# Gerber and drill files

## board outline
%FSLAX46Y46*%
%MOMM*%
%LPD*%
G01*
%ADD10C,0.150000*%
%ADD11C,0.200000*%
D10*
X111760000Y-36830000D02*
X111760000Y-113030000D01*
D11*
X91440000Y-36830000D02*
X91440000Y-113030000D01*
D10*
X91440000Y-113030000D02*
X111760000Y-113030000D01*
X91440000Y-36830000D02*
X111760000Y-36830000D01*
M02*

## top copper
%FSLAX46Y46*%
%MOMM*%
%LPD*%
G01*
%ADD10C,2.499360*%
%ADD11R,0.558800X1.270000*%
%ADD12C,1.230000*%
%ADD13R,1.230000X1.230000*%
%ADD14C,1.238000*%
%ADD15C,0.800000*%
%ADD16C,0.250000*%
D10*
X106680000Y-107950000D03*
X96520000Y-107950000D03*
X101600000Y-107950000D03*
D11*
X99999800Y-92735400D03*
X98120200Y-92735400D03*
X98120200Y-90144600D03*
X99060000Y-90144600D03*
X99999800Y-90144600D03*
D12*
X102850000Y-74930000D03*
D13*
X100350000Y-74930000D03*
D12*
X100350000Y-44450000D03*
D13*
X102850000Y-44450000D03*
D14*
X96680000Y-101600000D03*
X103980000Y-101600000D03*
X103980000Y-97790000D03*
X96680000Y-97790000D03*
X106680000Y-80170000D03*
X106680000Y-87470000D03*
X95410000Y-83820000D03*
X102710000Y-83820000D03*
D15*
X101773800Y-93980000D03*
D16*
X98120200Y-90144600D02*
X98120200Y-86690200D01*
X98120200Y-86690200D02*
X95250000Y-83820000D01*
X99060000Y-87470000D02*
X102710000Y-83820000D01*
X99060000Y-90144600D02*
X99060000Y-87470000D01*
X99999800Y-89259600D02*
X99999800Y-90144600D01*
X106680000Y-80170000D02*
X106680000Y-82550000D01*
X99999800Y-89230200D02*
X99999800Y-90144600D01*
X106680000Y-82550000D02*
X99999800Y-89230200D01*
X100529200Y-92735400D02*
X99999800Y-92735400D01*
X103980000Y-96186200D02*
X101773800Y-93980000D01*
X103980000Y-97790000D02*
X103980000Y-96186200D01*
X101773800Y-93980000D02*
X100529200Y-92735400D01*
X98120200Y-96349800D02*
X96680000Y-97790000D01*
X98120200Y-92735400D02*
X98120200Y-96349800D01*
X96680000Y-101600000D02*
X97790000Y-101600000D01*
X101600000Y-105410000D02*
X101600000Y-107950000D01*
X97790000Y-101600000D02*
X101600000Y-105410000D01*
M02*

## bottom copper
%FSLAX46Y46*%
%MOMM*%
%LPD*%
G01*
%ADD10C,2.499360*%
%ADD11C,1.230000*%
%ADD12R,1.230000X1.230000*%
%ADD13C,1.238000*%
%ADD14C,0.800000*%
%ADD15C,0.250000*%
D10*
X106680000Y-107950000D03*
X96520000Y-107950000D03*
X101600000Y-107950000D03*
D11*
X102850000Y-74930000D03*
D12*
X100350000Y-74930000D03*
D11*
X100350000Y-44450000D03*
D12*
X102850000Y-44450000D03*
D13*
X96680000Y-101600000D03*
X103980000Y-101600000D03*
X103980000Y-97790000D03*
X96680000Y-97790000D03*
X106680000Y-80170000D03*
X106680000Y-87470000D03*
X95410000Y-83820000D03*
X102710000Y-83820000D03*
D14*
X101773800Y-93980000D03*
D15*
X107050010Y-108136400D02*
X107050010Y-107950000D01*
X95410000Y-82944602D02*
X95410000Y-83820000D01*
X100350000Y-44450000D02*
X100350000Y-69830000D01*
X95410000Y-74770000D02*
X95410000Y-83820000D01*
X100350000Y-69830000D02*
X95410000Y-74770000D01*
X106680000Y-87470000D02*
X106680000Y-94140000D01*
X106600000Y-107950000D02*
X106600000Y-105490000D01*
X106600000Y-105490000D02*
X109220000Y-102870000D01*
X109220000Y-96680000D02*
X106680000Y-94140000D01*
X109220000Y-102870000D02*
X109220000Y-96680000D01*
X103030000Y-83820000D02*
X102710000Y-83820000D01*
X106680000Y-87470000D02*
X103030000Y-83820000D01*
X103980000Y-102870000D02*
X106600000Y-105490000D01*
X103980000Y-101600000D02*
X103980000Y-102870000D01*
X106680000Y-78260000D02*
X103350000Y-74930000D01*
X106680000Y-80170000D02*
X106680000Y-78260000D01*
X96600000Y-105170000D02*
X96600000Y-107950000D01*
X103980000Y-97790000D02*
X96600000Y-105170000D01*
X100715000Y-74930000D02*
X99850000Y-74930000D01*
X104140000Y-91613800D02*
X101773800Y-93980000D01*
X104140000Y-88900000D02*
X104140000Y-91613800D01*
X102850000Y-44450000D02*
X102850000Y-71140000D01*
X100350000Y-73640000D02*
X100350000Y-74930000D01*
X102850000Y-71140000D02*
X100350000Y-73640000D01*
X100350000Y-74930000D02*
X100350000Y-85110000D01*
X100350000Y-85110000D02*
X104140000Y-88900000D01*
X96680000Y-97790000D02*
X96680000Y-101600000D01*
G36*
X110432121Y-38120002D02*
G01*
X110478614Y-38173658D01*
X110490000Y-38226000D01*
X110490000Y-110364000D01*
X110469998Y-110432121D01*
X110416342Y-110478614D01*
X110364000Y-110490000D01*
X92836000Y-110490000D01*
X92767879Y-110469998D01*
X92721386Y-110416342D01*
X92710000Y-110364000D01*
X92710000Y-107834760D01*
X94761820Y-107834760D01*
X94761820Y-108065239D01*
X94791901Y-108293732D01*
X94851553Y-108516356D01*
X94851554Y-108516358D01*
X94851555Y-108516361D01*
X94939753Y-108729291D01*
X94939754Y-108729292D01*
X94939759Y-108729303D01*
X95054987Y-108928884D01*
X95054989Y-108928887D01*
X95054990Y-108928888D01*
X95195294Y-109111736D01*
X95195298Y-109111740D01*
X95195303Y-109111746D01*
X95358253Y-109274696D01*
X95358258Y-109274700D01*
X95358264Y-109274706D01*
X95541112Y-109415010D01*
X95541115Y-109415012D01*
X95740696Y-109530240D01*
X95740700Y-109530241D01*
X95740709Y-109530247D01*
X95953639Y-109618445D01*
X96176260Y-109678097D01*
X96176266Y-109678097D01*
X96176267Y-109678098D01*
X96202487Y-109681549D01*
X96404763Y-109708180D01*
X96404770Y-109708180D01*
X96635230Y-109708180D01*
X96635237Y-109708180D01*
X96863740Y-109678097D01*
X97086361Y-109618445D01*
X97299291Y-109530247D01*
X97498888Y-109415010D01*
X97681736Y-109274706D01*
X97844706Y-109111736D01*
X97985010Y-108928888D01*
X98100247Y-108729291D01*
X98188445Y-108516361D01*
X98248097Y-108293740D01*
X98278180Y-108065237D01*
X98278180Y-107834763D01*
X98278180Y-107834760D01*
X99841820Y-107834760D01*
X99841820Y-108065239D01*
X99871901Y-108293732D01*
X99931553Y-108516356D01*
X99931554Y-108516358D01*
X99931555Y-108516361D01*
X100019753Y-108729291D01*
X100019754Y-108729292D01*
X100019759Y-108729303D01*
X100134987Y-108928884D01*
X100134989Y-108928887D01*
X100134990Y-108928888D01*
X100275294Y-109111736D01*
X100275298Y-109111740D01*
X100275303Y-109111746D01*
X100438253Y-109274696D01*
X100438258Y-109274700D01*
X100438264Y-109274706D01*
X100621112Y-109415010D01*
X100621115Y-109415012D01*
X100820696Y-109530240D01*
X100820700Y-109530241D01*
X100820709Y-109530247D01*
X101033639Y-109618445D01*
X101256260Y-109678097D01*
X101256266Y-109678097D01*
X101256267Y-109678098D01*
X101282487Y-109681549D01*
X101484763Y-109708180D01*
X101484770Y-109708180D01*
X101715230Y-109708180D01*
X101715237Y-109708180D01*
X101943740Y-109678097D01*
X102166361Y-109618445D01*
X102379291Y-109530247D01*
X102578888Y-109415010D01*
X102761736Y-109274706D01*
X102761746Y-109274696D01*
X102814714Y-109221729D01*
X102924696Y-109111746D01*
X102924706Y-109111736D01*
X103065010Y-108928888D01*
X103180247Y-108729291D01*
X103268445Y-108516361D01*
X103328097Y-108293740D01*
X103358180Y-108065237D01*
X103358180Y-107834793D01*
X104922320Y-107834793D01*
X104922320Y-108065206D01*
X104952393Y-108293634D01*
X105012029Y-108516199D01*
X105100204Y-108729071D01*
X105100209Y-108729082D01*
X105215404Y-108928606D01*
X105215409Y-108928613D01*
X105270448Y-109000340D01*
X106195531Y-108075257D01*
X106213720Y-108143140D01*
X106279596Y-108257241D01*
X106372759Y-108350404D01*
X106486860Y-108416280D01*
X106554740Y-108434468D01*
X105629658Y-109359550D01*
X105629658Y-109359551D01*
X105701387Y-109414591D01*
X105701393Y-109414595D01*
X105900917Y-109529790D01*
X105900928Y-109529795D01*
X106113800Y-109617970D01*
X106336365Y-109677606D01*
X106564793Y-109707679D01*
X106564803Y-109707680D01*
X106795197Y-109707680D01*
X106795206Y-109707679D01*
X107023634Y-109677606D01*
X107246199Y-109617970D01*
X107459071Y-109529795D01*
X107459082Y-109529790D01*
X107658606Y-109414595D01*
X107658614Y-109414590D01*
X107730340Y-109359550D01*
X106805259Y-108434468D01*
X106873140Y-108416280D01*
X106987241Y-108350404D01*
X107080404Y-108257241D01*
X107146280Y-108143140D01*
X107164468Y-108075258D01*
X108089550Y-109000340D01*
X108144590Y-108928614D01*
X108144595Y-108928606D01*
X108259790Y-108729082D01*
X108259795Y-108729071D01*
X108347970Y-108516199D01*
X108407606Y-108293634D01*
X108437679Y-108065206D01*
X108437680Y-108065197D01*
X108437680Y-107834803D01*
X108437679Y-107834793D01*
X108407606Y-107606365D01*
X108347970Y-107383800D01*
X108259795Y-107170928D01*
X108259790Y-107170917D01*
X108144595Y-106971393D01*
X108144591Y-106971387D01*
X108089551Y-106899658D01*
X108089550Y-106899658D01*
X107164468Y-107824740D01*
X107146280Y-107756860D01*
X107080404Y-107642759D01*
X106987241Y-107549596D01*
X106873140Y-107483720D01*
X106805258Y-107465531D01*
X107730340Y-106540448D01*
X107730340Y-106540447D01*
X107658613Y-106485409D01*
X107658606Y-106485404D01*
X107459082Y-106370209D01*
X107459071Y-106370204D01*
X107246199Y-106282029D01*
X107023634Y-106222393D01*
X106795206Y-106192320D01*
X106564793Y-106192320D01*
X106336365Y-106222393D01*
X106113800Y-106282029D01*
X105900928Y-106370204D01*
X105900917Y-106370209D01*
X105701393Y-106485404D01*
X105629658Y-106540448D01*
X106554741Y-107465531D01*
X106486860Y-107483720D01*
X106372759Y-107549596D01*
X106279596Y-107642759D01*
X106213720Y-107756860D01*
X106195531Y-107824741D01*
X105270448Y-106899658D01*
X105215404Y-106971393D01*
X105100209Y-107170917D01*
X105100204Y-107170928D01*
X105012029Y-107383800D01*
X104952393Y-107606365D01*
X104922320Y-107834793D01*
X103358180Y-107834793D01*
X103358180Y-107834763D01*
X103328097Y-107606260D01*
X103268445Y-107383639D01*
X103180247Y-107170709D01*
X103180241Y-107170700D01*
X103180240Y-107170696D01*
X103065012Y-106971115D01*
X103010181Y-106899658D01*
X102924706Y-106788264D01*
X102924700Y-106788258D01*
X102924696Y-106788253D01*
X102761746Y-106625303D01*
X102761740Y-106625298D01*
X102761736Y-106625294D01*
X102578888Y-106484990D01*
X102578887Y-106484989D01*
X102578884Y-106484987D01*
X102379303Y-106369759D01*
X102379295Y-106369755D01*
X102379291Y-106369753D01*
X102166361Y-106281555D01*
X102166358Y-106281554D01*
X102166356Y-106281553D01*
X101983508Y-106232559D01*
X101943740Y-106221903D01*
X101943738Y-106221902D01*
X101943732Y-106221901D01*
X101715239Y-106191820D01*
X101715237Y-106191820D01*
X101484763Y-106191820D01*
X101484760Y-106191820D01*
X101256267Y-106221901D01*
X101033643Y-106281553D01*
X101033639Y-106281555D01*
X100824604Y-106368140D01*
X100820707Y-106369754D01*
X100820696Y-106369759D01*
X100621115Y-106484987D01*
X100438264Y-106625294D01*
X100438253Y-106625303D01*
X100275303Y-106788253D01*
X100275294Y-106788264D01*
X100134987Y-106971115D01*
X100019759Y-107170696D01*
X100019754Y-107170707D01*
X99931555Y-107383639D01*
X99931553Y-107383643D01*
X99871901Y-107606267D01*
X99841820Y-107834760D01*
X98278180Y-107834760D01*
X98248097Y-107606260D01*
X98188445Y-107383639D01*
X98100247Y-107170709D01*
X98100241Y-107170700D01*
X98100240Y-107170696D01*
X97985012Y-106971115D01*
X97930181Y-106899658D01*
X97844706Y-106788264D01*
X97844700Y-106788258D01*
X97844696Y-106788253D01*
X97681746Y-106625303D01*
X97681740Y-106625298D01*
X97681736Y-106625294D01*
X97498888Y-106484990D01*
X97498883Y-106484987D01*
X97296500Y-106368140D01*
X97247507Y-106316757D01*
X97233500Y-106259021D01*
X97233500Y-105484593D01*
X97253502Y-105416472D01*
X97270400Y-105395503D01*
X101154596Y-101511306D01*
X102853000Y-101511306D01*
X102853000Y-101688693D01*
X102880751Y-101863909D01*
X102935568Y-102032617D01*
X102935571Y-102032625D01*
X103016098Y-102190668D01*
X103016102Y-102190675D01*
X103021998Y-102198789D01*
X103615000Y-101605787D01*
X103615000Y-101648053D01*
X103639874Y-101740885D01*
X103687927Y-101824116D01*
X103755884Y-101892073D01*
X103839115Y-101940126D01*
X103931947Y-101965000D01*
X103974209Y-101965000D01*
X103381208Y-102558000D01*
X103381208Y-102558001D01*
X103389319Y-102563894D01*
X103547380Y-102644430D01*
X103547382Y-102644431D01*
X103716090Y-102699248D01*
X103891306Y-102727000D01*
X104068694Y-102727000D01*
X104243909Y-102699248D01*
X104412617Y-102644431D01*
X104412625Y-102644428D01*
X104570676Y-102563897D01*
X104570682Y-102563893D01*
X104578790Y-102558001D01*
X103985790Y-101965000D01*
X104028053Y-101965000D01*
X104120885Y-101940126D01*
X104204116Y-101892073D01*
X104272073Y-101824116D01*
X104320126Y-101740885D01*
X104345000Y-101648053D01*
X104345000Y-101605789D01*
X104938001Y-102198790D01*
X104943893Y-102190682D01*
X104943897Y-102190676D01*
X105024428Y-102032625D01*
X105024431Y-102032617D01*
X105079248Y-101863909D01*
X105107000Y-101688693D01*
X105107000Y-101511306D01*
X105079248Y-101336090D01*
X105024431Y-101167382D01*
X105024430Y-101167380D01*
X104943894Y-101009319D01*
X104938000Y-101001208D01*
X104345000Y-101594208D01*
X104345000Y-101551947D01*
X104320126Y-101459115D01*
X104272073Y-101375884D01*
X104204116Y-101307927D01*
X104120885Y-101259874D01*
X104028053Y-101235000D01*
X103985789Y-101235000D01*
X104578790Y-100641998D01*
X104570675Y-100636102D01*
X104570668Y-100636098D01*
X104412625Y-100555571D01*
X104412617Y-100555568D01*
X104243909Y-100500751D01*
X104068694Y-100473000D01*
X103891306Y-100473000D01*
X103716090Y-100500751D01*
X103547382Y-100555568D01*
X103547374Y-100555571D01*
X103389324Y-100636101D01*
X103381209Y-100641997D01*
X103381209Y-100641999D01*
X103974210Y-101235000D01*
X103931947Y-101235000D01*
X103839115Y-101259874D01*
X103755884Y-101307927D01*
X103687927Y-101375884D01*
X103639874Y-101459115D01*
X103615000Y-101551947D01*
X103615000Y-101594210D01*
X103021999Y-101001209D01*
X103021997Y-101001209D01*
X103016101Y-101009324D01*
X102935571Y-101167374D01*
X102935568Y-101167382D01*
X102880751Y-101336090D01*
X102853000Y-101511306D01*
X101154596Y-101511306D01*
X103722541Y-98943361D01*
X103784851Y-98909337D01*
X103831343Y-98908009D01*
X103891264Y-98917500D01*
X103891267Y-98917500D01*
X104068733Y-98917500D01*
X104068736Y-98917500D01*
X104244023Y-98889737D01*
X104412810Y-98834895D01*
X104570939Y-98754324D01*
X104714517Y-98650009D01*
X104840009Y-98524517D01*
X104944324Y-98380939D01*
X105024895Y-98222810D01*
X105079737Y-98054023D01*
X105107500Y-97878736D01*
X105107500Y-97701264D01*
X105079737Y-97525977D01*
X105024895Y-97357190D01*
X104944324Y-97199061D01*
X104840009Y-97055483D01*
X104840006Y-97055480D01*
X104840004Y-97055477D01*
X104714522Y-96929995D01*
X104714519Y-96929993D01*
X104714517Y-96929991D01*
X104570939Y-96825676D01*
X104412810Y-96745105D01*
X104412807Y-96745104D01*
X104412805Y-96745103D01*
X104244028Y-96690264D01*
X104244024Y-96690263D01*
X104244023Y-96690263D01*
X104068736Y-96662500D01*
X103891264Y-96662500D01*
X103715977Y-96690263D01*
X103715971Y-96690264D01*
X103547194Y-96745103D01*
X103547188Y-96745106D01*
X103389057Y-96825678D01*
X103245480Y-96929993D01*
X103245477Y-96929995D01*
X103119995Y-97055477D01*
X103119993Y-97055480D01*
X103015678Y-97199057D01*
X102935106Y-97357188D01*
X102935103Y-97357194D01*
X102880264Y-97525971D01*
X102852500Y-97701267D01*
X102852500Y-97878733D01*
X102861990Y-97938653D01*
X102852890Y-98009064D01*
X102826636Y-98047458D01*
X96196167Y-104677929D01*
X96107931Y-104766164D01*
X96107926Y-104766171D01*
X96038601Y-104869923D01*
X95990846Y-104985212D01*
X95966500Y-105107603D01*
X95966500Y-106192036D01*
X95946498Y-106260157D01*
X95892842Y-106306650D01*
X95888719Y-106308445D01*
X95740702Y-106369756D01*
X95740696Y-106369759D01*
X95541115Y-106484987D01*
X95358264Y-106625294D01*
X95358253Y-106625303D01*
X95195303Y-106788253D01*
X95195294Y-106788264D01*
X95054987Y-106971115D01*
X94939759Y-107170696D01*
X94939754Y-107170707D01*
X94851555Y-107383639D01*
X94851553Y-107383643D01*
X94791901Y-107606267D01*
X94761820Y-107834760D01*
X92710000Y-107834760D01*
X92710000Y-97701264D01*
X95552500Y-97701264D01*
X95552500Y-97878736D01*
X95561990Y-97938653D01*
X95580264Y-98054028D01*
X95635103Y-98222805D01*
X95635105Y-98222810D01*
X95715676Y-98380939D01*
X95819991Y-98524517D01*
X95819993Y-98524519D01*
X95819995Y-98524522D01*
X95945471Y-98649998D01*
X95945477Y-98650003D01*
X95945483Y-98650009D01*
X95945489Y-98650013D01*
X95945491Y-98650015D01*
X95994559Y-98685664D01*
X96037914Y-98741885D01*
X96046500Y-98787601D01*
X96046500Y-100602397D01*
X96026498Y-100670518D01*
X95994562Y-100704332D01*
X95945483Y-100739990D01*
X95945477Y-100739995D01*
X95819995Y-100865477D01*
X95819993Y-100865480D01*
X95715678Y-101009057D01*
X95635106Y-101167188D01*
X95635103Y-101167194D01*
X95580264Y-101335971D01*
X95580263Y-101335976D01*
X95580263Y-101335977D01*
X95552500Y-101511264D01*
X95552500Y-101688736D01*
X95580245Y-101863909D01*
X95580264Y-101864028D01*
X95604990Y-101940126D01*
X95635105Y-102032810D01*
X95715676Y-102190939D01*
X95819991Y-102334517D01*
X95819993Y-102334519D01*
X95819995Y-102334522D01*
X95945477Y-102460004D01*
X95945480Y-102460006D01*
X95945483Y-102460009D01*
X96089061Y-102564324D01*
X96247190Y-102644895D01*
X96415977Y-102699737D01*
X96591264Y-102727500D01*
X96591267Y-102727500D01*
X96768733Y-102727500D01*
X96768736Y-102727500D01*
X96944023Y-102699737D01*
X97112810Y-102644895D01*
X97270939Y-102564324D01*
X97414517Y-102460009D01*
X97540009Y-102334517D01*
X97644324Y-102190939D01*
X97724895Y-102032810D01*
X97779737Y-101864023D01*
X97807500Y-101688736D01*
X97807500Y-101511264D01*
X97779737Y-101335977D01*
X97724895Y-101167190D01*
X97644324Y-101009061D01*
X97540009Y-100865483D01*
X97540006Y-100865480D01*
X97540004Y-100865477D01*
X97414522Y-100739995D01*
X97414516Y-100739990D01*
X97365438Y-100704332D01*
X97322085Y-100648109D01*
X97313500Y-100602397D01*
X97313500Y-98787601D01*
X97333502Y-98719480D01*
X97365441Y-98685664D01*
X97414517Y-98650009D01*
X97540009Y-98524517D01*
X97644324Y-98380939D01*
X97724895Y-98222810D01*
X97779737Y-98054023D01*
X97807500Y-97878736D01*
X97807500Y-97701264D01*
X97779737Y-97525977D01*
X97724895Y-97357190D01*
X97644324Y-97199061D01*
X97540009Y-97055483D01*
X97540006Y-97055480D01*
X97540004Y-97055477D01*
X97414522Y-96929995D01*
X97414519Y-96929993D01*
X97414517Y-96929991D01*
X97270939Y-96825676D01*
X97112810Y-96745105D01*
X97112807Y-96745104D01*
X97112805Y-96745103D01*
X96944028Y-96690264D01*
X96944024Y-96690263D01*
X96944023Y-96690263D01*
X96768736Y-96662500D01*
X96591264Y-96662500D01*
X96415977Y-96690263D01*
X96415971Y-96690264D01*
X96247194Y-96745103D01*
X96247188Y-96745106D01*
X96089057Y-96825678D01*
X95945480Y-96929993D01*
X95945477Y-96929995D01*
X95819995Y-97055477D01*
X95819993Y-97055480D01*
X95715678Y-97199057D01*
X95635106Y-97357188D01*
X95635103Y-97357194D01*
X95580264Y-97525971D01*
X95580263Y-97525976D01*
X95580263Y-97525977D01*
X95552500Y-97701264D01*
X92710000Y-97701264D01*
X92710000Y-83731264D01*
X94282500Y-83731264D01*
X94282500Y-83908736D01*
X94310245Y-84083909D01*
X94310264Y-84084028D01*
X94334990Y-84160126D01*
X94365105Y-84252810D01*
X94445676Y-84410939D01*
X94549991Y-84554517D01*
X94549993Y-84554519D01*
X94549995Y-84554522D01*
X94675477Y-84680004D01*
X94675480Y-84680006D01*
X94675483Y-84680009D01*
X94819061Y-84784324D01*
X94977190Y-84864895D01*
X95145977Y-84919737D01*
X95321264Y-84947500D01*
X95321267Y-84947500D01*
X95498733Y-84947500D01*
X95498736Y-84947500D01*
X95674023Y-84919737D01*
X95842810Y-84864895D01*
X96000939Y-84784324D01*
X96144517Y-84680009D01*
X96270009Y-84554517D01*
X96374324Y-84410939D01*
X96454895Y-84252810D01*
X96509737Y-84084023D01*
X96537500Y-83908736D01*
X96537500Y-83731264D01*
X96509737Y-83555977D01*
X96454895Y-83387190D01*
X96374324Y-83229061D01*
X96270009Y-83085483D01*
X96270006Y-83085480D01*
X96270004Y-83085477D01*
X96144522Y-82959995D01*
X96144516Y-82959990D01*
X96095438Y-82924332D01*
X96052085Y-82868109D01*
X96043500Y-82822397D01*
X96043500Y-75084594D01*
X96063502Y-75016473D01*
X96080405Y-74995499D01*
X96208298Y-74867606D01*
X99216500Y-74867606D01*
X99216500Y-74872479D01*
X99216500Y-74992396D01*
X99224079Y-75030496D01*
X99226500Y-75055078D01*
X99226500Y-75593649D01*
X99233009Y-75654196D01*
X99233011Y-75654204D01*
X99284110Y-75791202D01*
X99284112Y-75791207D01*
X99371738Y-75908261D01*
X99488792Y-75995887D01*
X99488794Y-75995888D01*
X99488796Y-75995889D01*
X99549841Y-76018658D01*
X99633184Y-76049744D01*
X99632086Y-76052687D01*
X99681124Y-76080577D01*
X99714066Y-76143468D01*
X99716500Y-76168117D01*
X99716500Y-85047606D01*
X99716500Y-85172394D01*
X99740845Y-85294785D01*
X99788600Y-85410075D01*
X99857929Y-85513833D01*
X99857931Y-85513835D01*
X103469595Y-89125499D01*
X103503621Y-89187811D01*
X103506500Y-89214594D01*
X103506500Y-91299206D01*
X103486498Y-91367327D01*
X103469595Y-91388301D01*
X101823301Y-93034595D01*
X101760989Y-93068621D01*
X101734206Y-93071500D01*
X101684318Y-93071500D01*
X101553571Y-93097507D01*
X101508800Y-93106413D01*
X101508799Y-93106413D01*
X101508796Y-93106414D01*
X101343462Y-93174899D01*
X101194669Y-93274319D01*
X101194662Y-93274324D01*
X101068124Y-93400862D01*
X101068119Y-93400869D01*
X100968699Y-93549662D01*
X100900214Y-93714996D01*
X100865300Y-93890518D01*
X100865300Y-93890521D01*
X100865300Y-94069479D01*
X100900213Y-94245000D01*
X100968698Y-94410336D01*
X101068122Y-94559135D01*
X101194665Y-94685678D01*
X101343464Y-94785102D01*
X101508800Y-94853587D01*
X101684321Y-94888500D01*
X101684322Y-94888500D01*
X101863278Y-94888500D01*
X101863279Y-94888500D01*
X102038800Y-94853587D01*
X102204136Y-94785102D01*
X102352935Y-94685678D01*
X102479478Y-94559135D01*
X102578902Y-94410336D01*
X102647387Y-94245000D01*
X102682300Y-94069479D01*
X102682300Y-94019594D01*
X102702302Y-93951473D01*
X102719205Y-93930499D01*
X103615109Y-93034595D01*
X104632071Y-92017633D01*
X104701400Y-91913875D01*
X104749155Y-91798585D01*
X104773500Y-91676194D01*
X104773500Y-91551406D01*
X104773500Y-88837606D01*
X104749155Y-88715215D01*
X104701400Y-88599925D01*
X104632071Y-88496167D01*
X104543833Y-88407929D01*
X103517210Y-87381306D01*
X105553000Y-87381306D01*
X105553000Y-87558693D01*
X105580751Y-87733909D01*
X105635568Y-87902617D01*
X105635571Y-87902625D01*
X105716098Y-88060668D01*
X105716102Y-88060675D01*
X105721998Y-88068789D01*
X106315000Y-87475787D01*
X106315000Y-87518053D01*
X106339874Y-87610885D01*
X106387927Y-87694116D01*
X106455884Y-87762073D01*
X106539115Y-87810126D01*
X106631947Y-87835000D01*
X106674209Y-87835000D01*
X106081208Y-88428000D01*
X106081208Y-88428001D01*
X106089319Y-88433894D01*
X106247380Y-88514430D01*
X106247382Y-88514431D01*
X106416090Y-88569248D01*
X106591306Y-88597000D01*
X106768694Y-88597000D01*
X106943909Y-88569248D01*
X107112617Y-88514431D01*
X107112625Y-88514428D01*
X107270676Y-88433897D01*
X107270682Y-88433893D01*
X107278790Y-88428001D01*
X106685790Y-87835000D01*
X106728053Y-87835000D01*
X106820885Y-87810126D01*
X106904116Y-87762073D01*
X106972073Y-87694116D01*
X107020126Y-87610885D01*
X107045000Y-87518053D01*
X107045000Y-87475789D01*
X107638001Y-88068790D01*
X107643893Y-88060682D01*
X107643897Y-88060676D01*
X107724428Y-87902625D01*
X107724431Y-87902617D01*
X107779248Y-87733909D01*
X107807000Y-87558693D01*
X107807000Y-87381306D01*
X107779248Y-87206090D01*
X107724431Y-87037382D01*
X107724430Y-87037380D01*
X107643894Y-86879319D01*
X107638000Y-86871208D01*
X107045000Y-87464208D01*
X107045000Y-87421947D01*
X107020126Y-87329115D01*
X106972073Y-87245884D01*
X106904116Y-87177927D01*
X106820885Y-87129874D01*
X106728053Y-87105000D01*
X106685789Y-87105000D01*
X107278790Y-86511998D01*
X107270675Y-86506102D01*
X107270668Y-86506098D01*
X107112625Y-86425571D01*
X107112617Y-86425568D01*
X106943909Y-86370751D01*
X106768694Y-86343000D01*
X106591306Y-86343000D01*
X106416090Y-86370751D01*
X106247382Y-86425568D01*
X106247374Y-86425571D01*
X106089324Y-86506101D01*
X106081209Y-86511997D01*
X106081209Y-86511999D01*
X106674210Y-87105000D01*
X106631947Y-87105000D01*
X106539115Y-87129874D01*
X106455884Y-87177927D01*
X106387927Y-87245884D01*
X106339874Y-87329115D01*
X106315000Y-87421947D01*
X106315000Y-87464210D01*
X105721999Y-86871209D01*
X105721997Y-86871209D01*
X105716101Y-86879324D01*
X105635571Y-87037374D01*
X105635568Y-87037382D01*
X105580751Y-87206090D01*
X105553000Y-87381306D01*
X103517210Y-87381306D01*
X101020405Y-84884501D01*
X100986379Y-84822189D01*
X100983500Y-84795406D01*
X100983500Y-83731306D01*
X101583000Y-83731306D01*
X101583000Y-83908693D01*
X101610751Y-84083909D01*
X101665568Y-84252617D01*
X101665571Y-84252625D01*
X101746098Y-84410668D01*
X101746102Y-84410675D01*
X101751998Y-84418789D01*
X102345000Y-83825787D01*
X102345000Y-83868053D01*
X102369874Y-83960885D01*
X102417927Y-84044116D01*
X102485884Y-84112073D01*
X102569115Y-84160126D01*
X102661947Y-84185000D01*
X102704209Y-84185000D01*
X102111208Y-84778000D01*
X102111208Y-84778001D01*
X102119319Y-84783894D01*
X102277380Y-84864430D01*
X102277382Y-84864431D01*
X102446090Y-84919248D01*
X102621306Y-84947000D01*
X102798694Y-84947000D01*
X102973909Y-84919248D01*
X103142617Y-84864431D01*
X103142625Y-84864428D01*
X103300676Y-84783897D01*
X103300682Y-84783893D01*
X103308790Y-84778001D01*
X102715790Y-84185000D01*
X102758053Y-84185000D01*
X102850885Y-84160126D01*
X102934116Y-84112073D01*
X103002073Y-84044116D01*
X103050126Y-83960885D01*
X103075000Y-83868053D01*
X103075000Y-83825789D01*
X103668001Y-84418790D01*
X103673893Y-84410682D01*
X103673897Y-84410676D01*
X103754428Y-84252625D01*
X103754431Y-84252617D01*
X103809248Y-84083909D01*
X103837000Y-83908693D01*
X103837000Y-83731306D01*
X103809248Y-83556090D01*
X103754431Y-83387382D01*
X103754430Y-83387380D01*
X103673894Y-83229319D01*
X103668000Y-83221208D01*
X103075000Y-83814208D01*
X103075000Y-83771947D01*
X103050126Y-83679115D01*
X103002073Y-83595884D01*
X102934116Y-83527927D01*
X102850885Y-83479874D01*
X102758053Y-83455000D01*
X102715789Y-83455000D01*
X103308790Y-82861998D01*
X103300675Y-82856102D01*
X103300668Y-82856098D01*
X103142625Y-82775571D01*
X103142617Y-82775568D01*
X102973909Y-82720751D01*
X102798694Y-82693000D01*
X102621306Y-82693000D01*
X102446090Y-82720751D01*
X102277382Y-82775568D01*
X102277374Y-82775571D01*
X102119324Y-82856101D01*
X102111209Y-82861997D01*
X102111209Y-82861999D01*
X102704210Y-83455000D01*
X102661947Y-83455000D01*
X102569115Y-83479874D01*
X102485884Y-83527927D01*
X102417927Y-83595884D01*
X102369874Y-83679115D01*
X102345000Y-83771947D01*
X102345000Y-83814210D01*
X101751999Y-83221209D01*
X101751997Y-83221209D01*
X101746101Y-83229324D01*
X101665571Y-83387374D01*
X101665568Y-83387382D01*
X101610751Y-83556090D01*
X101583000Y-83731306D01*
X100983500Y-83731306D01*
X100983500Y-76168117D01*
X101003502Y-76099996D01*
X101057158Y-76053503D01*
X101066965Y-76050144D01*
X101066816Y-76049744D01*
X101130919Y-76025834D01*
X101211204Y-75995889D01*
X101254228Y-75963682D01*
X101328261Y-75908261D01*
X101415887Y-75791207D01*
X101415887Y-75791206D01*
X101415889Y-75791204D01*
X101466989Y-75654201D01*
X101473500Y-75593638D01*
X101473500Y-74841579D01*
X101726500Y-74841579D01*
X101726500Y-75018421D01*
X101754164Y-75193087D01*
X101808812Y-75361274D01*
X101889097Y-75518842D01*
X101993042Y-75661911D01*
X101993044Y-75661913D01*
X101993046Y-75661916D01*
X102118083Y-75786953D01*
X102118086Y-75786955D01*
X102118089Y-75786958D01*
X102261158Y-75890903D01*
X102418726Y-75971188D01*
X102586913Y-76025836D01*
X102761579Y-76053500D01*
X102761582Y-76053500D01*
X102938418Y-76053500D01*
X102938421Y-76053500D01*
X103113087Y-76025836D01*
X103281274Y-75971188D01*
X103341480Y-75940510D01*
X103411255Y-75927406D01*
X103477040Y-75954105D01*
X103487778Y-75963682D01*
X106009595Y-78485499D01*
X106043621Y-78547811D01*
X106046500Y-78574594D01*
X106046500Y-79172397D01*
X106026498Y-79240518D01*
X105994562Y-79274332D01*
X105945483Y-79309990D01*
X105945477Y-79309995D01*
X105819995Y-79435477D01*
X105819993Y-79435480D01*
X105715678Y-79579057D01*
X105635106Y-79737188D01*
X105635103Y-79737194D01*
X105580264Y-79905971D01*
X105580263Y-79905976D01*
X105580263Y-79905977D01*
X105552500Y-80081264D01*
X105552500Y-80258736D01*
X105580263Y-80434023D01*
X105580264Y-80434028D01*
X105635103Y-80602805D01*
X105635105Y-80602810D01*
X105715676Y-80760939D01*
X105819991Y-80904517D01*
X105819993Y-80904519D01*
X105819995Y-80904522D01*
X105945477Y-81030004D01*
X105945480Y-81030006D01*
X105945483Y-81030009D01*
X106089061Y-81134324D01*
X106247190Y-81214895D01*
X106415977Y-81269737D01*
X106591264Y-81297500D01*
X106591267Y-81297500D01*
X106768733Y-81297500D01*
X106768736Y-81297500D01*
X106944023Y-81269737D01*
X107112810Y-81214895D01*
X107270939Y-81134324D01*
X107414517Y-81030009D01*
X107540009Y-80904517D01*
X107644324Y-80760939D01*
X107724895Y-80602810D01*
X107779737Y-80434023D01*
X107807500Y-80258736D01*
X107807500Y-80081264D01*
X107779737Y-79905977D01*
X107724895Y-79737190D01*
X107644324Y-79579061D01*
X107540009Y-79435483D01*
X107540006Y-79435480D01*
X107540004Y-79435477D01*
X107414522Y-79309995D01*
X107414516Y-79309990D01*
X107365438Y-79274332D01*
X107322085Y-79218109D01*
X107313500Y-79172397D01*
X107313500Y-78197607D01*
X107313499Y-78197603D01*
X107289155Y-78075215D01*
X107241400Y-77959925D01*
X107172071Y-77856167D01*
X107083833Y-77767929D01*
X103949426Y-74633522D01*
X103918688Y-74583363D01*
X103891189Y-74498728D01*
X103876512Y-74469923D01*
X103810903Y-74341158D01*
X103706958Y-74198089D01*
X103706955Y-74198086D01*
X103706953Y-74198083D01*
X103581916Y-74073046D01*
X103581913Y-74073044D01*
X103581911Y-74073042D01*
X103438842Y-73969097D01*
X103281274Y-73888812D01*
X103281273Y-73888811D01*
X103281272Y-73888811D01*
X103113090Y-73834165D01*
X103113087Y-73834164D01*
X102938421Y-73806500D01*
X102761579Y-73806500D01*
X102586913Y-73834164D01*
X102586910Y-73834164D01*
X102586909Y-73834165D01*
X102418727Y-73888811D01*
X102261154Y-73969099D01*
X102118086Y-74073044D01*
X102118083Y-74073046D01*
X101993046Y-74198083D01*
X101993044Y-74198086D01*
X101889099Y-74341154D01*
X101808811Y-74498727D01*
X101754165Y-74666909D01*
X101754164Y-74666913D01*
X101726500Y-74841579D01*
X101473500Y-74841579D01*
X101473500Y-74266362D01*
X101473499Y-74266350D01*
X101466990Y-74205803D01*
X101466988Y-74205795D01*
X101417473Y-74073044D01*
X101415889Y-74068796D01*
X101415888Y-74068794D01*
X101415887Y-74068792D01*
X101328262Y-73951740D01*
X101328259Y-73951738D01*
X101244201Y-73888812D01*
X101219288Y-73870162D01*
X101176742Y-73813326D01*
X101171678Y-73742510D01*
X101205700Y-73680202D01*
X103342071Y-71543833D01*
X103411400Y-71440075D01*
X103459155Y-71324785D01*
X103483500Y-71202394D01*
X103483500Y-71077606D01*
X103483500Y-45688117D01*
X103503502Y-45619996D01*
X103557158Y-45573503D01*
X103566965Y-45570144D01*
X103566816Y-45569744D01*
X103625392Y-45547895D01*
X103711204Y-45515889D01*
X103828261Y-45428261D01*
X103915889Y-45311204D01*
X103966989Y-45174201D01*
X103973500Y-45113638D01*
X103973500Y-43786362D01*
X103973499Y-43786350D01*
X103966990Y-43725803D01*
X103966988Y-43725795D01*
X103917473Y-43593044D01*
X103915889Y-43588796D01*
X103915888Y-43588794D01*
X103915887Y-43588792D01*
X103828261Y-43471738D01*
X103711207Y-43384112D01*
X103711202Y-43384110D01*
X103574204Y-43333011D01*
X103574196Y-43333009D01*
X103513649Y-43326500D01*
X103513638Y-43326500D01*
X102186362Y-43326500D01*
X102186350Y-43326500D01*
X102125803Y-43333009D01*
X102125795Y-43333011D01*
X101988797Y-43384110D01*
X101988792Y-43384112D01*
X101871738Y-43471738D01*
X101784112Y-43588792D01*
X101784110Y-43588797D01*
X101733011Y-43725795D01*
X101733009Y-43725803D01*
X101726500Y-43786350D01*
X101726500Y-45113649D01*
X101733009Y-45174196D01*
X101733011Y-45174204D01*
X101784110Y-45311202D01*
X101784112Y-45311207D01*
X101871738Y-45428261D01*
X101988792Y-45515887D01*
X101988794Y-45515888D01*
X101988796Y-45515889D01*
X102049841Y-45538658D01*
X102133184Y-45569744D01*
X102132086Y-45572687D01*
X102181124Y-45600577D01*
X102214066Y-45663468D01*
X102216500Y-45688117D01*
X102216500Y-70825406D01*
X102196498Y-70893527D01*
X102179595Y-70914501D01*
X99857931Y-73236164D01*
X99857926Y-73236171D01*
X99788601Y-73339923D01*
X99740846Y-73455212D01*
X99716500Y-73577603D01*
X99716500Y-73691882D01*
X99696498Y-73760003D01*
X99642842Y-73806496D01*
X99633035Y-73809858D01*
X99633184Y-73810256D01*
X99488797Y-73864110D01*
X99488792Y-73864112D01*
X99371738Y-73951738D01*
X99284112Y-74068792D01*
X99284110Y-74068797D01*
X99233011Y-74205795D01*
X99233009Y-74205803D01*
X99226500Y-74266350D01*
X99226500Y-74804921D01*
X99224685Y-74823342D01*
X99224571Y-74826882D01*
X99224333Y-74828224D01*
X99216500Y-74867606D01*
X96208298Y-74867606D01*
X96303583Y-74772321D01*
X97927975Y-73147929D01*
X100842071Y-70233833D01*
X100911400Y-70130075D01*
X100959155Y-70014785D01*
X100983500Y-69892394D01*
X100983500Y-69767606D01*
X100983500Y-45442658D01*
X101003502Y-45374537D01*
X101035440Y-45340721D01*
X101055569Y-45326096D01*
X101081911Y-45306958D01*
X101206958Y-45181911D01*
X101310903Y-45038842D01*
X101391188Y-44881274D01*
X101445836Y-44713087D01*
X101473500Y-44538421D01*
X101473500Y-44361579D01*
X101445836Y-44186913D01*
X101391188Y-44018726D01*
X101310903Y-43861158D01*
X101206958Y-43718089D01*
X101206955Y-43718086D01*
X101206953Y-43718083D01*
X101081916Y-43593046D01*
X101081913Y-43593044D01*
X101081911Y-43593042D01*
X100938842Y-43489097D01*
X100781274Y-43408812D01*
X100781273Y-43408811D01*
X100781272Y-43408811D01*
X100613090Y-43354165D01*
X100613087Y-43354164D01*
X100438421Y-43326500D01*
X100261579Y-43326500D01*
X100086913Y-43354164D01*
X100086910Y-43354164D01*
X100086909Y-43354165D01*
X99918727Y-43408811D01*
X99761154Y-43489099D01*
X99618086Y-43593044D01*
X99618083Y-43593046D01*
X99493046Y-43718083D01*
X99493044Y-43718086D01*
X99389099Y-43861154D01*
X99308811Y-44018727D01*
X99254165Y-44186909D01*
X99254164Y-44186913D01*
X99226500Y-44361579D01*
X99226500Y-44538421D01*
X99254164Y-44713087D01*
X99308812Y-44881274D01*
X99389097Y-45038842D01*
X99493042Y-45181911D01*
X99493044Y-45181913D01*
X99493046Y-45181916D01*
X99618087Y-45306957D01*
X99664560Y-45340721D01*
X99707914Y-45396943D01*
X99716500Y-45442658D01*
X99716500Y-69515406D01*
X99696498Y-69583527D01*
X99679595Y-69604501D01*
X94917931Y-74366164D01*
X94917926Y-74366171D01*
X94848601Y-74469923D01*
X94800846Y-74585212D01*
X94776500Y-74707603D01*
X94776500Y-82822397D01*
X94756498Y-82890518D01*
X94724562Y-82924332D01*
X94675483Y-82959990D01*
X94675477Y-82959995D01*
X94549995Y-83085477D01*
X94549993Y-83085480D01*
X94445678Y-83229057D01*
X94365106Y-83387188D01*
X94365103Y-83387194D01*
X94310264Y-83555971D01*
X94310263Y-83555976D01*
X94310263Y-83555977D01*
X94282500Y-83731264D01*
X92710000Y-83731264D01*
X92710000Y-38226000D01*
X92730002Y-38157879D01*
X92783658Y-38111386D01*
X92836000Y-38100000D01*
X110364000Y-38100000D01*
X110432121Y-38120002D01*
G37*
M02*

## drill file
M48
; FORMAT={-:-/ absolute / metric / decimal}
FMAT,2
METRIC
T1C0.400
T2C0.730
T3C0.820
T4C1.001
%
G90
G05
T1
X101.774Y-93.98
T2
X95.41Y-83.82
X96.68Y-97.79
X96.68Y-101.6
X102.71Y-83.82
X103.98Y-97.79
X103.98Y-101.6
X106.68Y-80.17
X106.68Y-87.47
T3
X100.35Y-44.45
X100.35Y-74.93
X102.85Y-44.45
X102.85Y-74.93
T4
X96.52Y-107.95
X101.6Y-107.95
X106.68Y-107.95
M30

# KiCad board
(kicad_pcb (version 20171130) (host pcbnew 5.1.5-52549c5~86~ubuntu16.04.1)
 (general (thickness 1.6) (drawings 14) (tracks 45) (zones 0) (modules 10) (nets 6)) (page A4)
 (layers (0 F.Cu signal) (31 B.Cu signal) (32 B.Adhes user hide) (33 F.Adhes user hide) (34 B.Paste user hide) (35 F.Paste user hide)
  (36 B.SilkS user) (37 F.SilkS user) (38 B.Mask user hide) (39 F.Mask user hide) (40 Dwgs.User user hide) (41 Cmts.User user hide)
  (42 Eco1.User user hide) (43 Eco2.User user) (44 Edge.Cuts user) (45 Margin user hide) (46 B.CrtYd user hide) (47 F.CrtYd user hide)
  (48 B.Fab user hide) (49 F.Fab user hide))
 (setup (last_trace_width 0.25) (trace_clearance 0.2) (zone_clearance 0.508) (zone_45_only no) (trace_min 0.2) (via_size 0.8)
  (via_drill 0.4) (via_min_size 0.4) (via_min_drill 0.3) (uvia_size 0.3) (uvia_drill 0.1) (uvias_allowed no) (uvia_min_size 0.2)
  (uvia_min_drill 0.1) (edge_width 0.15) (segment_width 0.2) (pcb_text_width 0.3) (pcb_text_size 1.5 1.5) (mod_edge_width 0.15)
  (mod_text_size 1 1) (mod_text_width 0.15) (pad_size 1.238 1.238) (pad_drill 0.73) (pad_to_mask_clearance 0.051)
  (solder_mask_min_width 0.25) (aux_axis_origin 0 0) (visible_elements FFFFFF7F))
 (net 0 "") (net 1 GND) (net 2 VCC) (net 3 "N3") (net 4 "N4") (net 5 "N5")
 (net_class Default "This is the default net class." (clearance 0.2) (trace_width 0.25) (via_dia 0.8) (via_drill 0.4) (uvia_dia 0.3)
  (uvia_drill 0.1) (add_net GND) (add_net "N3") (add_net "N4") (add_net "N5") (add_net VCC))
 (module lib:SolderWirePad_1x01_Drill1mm (layer F.Cu) (at 106.68 107.95)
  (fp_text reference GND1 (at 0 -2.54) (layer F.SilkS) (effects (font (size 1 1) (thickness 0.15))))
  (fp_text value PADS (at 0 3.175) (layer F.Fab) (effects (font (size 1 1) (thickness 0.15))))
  (pad 1 thru_hole circle (at 0 0) (size 2.49936 2.49936) (drill 1.00076) (layers *.Cu *.Mask) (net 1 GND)))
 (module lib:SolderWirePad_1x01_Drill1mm (layer F.Cu) (at 96.52 107.95)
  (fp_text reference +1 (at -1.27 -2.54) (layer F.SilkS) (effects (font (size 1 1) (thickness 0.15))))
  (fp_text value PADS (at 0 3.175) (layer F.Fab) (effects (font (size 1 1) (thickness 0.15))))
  (pad 1 thru_hole circle (at 0 0) (size 2.49936 2.49936) (drill 1.00076) (layers *.Cu *.Mask) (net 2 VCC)))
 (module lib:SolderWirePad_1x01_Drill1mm (layer F.Cu) (at 101.6 107.95)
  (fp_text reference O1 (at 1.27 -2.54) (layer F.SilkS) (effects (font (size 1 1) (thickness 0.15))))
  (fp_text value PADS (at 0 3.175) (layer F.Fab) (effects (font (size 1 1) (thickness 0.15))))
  (pad 1 thru_hole circle (at 0 0) (size 2.49936 2.49936) (drill 1.00076) (layers *.Cu *.Mask) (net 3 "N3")))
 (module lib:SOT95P (layer F.Cu) (at 99.06 91.44 270)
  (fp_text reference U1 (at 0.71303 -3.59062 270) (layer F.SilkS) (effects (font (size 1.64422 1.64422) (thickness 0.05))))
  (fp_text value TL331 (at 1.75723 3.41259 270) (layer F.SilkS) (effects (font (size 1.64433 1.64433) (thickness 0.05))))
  (pad 5 smd rect (at 1.2954 -0.9398 270) (size 1.27 0.5588) (layers F.Cu F.Paste F.Mask) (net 2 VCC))
  (pad 4 smd rect (at 1.2954 0.9398 270) (size 1.27 0.5588) (layers F.Cu F.Paste F.Mask) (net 3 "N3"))
  (pad 3 smd rect (at -1.2954 0.9398 270) (size 1.27 0.5588) (layers F.Cu F.Paste F.Mask) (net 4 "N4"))
  (pad 2 smd rect (at -1.2954 0 270) (size 1.27 0.5588) (layers F.Cu F.Paste F.Mask) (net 1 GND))
  (pad 1 smd rect (at -1.2954 -0.9398 270) (size 1.27 0.5588) (layers F.Cu F.Paste F.Mask) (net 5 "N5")))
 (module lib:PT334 (layer F.Cu) (at 101.6 74.93)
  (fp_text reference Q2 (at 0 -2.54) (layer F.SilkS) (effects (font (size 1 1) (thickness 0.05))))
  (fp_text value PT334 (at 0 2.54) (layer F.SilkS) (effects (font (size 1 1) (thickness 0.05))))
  (pad E thru_hole circle (at 1.25 0) (size 1.23 1.23) (drill 0.82) (layers *.Cu *.Mask) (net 5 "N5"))
  (pad C thru_hole rect (at -1.25 0) (size 1.23 1.23) (drill 0.82) (layers *.Cu *.Mask) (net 2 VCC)))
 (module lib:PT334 (layer F.Cu) (at 101.6 44.45 180)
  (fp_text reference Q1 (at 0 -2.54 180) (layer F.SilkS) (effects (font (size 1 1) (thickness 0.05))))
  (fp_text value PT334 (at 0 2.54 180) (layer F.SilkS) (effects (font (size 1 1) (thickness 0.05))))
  (pad E thru_hole circle (at 1.25 0 180) (size 1.23 1.23) (drill 0.82) (layers *.Cu *.Mask) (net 4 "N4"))
  (pad C thru_hole rect (at -1.25 0 180) (size 1.23 1.23) (drill 0.82) (layers *.Cu *.Mask) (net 2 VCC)))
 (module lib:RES (layer F.Cu) (at 100.33 101.6 180)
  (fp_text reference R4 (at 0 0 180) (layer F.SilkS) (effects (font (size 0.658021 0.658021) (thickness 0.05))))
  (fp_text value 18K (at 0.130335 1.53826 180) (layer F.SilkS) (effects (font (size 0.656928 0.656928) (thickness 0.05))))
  (pad 2 thru_hole circle (at 3.65 0 180) (size 1.238 1.238) (drill 0.73) (layers *.Cu *.Mask) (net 3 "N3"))
  (pad 1 thru_hole circle (at -3.65 0 180) (size 1.238 1.238) (drill 0.73) (layers *.Cu *.Mask) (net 1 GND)))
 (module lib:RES (layer F.Cu) (at 100.33 97.79)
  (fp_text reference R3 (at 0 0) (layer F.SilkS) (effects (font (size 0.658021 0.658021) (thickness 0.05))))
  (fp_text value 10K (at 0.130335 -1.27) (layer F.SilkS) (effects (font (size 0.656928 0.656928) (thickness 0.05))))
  (pad 2 thru_hole circle (at 3.65 0) (size 1.238 1.238) (drill 0.73) (layers *.Cu *.Mask) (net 2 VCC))
  (pad 1 thru_hole circle (at -3.65 0) (size 1.238 1.238) (drill 0.73) (layers *.Cu *.Mask) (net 3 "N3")))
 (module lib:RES (layer F.Cu) (at 106.68 83.82 90)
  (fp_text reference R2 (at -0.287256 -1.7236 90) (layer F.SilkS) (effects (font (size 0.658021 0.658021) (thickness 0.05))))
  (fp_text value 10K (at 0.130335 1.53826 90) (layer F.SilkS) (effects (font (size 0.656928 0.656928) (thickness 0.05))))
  (pad 2 thru_hole circle (at 3.65 0 90) (size 1.238 1.238) (drill 0.73) (layers *.Cu *.Mask) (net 5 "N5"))
  (pad 1 thru_hole circle (at -3.65 0 90) (size 1.238 1.238) (drill 0.73) (layers *.Cu *.Mask) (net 1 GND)))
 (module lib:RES (layer F.Cu) (at 99.06 83.82 180)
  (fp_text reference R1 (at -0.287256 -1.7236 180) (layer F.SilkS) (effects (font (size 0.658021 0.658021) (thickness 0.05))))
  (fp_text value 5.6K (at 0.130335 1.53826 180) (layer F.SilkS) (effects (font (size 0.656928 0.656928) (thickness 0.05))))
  (pad 2 thru_hole circle (at 3.65 0 180) (size 1.238 1.238) (drill 0.73) (layers *.Cu *.Mask) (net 4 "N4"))
  (pad 1 thru_hole circle (at -3.65 0 180) (size 1.238 1.238) (drill 0.73) (layers *.Cu *.Mask) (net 1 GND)))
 (gr_line (start 111.76 36.83) (end 111.76 113.03) (layer Edge.Cuts) (width 0.15))
 (gr_line (start 91.44 36.83) (end 91.44 113.03) (layer Edge.Cuts) (width 0.2))
 (gr_line (start 91.44 113.03) (end 111.76 113.03) (layer Edge.Cuts) (width 0.15))
 (gr_line (start 91.44 36.83) (end 111.76 36.83) (layer Edge.Cuts) (width 0.15))
 (segment (start 107.05001 108.1364) (end 107.05001 107.95) (width 0.25) (layer B.Cu) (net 1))
 (segment (start 95.41 82.944602) (end 95.41 83.82) (width 0.25) (layer B.Cu) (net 4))
 (segment (start 98.1202 90.1446) (end 98.1202 86.6902) (width 0.25) (layer F.Cu) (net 4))
 (segment (start 98.1202 86.6902) (end 95.25 83.82) (width 0.25) (layer F.Cu) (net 4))
 (segment (start 100.35 44.45) (end 100.35 69.83) (width 0.25) (layer B.Cu) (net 4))
 (segment (start 95.41 74.77) (end 95.41 83.82) (width 0.25) (layer B.Cu) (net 4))
 (segment (start 100.35 69.83) (end 95.41 74.77) (width 0.25) (layer B.Cu) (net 4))
 (segment (start 106.68 87.47) (end 106.68 94.14) (width 0.25) (layer B.Cu) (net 1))
 (segment (start 106.6 107.95) (end 106.6 105.49) (width 0.25) (layer B.Cu) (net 1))
 (segment (start 106.6 105.49) (end 109.22 102.87) (width 0.25) (layer B.Cu) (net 1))
 (segment (start 109.22 96.68) (end 106.68 94.14) (width 0.25) (layer B.Cu) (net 1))
 (segment (start 109.22 102.87) (end 109.22 96.68) (width 0.25) (layer B.Cu) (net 1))
 (segment (start 103.03 83.82) (end 102.71 83.82) (width 0.25) (layer B.Cu) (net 1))
 (segment (start 106.68 87.47) (end 103.03 83.82) (width 0.25) (layer B.Cu) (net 1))
 (segment (start 99.06 87.47) (end 102.71 83.82) (width 0.25) (layer F.Cu) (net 1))
 (segment (start 99.06 90.1446) (end 99.06 87.47) (width 0.25) (layer F.Cu) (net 1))
 (segment (start 103.98 102.87) (end 106.6 105.49) (width 0.25) (layer B.Cu) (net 1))
 (segment (start 103.98 101.6) (end 103.98 102.87) (width 0.25) (layer B.Cu) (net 1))
 (segment (start 106.68 78.26) (end 103.35 74.93) (width 0.25) (layer B.Cu) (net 5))
 (segment (start 106.68 80.17) (end 106.68 78.26) (width 0.25) (layer B.Cu) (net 5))
 (segment (start 99.9998 89.2596) (end 99.9998 90.1446) (width 0.25) (layer F.Cu) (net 5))
 (segment (start 106.68 80.17) (end 106.68 82.55) (width 0.25) (layer F.Cu) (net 5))
 (segment (start 99.9998 89.2302) (end 99.9998 90.1446) (width 0.25) (layer F.Cu) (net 5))
 (segment (start 106.68 82.55) (end 99.9998 89.2302) (width 0.25) (layer F.Cu) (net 5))
 (segment (start 96.6 105.17) (end 96.6 107.95) (width 0.25) (layer B.Cu) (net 2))
 (segment (start 103.98 97.79) (end 96.6 105.17) (width 0.25) (layer B.Cu) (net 2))
 (segment (start 100.5292 92.7354) (end 99.9998 92.7354) (width 0.25) (layer F.Cu) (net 2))
 (segment (start 103.98 96.1862) (end 101.7738 93.98) (width 0.25) (layer F.Cu) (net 2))
 (segment (start 103.98 97.79) (end 103.98 96.1862) (width 0.25) (layer F.Cu) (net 2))
 (segment (start 100.715 74.93) (end 99.85 74.93) (width 0.25) (layer B.Cu) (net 2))
 (segment (start 101.7738 93.98) (end 100.5292 92.7354) (width 0.25) (layer F.Cu) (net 2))
 (via (at 101.7738 93.98) (size 0.8) (drill 0.4) (layers F.Cu B.Cu) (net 2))
 (segment (start 104.14 91.6138) (end 101.7738 93.98) (width 0.25) (layer B.Cu) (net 2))
 (segment (start 104.14 88.9) (end 104.14 91.6138) (width 0.25) (layer B.Cu) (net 2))
 (segment (start 102.85 44.45) (end 102.85 71.14) (width 0.25) (layer B.Cu) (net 2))
 (segment (start 100.35 73.64) (end 100.35 74.93) (width 0.25) (layer B.Cu) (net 2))
 (segment (start 102.85 71.14) (end 100.35 73.64) (width 0.25) (layer B.Cu) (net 2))
 (segment (start 100.35 74.93) (end 100.35 85.11) (width 0.25) (layer B.Cu) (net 2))
 (segment (start 100.35 85.11) (end 104.14 88.9) (width 0.25) (layer B.Cu) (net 2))
 (segment (start 98.1202 96.3498) (end 96.68 97.79) (width 0.25) (layer F.Cu) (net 3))
 (segment (start 98.1202 92.7354) (end 98.1202 96.3498) (width 0.25) (layer F.Cu) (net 3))
 (segment (start 96.68 97.79) (end 96.68 101.6) (width 0.25) (layer B.Cu) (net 3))
 (segment (start 96.68 101.6) (end 97.79 101.6) (width 0.25) (layer F.Cu) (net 3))
 (segment (start 101.6 105.41) (end 101.6 107.95) (width 0.25) (layer F.Cu) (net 3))
 (segment (start 97.79 101.6) (end 101.6 105.41) (width 0.25) (layer F.Cu) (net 3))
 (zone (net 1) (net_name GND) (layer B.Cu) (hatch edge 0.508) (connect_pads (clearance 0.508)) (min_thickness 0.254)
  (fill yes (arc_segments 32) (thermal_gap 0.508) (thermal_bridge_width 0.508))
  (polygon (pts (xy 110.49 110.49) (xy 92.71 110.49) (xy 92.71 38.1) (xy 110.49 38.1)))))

